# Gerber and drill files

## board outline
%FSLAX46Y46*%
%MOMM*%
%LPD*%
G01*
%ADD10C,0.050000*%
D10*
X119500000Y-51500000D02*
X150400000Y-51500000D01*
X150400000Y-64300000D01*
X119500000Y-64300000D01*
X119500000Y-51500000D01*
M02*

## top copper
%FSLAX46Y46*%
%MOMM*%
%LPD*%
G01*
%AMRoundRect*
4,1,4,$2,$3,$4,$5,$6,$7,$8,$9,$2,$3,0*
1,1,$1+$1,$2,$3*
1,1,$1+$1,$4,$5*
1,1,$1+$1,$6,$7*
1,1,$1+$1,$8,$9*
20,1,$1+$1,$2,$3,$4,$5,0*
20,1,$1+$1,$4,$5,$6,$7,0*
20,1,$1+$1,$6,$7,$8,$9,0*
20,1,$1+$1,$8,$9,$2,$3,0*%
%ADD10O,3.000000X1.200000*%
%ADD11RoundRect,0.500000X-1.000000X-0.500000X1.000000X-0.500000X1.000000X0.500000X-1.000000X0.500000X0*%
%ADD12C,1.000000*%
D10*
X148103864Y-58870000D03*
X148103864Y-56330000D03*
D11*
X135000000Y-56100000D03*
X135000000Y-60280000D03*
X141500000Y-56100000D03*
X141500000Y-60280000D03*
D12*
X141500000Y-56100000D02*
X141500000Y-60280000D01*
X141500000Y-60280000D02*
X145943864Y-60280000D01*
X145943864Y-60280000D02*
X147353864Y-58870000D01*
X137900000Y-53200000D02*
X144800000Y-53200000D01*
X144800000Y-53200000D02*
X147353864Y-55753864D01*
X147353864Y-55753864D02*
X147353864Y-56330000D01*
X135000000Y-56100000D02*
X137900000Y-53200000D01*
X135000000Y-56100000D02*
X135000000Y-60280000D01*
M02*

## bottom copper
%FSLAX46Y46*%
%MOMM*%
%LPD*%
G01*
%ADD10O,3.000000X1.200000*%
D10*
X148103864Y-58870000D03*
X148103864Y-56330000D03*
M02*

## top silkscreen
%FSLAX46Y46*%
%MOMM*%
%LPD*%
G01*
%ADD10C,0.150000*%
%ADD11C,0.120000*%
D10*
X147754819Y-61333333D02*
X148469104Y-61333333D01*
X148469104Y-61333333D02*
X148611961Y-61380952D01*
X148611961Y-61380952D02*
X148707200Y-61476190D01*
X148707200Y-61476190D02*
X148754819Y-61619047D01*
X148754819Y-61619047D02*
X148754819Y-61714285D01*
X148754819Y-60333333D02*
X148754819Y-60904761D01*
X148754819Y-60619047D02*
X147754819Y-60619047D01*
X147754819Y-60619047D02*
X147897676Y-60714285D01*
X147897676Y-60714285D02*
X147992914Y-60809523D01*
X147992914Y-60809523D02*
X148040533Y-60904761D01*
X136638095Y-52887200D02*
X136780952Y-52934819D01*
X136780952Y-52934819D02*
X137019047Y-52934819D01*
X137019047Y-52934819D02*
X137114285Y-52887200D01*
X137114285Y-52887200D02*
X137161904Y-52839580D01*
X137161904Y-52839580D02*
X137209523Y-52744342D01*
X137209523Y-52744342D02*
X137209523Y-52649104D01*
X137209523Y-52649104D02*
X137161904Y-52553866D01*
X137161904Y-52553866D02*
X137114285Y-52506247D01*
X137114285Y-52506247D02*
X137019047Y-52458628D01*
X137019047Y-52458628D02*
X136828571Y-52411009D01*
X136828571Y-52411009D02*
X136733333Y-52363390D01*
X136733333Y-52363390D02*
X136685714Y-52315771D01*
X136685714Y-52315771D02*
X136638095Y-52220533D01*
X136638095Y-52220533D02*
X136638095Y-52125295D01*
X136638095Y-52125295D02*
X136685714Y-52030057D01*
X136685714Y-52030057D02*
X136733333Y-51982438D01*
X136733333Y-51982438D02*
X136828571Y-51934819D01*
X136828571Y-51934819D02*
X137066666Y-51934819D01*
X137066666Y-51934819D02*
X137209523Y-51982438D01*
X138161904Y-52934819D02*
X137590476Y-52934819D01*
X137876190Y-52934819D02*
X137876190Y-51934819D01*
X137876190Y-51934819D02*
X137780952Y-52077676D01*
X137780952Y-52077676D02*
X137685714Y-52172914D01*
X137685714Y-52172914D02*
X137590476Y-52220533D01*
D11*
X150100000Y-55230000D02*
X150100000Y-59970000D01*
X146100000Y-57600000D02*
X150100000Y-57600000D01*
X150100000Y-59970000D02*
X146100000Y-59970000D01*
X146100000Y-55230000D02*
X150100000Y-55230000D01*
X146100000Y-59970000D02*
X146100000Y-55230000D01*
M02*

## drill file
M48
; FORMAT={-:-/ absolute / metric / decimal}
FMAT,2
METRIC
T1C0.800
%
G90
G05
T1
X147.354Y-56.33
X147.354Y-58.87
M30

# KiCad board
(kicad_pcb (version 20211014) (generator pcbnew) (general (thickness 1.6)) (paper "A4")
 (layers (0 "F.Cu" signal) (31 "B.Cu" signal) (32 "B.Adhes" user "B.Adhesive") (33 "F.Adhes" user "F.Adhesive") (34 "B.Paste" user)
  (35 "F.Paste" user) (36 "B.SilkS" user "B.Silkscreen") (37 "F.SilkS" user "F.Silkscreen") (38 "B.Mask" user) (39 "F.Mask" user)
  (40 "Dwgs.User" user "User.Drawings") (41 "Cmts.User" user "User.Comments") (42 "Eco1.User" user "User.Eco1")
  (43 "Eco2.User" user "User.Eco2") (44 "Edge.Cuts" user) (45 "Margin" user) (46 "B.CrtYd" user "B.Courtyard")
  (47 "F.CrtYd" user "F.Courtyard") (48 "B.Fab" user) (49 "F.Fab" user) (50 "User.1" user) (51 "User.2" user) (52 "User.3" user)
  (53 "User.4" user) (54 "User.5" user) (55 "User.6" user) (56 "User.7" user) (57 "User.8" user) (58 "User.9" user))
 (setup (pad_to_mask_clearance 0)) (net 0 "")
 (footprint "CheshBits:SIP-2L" (layer "F.Cu") (at 148.1 57.6 90)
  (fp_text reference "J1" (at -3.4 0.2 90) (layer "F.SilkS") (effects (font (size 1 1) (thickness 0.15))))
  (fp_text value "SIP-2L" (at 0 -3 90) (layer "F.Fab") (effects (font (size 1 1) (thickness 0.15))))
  (fp_line (start 2.37 2) (end -2.37 2) (layer "F.SilkS") (width 0.12))
  (fp_line (start 0 -2) (end 0 2) (layer "F.SilkS") (width 0.12))
  (fp_line (start -2.37 2) (end -2.37 -2) (layer "F.SilkS") (width 0.12))
  (fp_line (start 2.37 -2) (end 2.37 2) (layer "F.SilkS") (width 0.12))
  (fp_line (start -2.37 -2) (end 2.37 -2) (layer "F.SilkS") (width 0.12))
  (pad "1" thru_hole oval (at -1.27 -0.746136 90) (size 1.2 3) (drill 0.8 (offset 0 0.75)) (layers *.Cu *.Mask))
  (pad "2" thru_hole oval (at 1.27 -0.746136 90) (size 1.2 3) (drill 0.8 (offset 0 0.75)) (layers *.Cu *.Mask)))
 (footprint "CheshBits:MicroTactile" (layer "F.Cu") (at 137.4 52.98)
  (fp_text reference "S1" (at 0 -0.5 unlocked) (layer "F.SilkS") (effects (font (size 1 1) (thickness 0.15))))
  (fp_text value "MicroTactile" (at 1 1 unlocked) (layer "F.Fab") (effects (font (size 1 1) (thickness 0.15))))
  (pad "1" smd roundrect (at -2.4 3.12) (size 3 2) (layers "F.Cu" "F.Paste" "F.Mask") (roundrect_rratio 0.25))
  (pad "2" smd roundrect (at -2.4 7.3) (size 3 2) (layers "F.Cu" "F.Paste" "F.Mask") (roundrect_rratio 0.25))
  (pad "3" smd roundrect (at 4.1 3.12) (size 3 2) (layers "F.Cu" "F.Paste" "F.Mask") (roundrect_rratio 0.25))
  (pad "4" smd roundrect (at 4.1 7.3) (size 3 2) (layers "F.Cu" "F.Paste" "F.Mask") (roundrect_rratio 0.25)))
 (gr_rect (start 119.5 51.5) (end 150.4 64.3) (layer "Edge.Cuts") (width 0.05) (fill none))
 (segment (start 141.5 56.1) (end 141.5 60.28) (width 1) (layer "F.Cu") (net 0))
 (segment (start 141.5 60.28) (end 145.943864 60.28) (width 1) (layer "F.Cu") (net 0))
 (segment (start 145.943864 60.28) (end 147.353864 58.87) (width 1) (layer "F.Cu") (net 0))
 (segment (start 137.9 53.2) (end 144.8 53.2) (width 1) (layer "F.Cu") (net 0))
 (segment (start 144.8 53.2) (end 147.353864 55.753864) (width 1) (layer "F.Cu") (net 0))
 (segment (start 147.353864 55.753864) (end 147.353864 56.33) (width 1) (layer "F.Cu") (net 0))
 (segment (start 135 56.1) (end 137.9 53.2) (width 1) (layer "F.Cu") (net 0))
 (segment (start 135 56.1) (end 135 60.28) (width 1) (layer "F.Cu") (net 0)))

